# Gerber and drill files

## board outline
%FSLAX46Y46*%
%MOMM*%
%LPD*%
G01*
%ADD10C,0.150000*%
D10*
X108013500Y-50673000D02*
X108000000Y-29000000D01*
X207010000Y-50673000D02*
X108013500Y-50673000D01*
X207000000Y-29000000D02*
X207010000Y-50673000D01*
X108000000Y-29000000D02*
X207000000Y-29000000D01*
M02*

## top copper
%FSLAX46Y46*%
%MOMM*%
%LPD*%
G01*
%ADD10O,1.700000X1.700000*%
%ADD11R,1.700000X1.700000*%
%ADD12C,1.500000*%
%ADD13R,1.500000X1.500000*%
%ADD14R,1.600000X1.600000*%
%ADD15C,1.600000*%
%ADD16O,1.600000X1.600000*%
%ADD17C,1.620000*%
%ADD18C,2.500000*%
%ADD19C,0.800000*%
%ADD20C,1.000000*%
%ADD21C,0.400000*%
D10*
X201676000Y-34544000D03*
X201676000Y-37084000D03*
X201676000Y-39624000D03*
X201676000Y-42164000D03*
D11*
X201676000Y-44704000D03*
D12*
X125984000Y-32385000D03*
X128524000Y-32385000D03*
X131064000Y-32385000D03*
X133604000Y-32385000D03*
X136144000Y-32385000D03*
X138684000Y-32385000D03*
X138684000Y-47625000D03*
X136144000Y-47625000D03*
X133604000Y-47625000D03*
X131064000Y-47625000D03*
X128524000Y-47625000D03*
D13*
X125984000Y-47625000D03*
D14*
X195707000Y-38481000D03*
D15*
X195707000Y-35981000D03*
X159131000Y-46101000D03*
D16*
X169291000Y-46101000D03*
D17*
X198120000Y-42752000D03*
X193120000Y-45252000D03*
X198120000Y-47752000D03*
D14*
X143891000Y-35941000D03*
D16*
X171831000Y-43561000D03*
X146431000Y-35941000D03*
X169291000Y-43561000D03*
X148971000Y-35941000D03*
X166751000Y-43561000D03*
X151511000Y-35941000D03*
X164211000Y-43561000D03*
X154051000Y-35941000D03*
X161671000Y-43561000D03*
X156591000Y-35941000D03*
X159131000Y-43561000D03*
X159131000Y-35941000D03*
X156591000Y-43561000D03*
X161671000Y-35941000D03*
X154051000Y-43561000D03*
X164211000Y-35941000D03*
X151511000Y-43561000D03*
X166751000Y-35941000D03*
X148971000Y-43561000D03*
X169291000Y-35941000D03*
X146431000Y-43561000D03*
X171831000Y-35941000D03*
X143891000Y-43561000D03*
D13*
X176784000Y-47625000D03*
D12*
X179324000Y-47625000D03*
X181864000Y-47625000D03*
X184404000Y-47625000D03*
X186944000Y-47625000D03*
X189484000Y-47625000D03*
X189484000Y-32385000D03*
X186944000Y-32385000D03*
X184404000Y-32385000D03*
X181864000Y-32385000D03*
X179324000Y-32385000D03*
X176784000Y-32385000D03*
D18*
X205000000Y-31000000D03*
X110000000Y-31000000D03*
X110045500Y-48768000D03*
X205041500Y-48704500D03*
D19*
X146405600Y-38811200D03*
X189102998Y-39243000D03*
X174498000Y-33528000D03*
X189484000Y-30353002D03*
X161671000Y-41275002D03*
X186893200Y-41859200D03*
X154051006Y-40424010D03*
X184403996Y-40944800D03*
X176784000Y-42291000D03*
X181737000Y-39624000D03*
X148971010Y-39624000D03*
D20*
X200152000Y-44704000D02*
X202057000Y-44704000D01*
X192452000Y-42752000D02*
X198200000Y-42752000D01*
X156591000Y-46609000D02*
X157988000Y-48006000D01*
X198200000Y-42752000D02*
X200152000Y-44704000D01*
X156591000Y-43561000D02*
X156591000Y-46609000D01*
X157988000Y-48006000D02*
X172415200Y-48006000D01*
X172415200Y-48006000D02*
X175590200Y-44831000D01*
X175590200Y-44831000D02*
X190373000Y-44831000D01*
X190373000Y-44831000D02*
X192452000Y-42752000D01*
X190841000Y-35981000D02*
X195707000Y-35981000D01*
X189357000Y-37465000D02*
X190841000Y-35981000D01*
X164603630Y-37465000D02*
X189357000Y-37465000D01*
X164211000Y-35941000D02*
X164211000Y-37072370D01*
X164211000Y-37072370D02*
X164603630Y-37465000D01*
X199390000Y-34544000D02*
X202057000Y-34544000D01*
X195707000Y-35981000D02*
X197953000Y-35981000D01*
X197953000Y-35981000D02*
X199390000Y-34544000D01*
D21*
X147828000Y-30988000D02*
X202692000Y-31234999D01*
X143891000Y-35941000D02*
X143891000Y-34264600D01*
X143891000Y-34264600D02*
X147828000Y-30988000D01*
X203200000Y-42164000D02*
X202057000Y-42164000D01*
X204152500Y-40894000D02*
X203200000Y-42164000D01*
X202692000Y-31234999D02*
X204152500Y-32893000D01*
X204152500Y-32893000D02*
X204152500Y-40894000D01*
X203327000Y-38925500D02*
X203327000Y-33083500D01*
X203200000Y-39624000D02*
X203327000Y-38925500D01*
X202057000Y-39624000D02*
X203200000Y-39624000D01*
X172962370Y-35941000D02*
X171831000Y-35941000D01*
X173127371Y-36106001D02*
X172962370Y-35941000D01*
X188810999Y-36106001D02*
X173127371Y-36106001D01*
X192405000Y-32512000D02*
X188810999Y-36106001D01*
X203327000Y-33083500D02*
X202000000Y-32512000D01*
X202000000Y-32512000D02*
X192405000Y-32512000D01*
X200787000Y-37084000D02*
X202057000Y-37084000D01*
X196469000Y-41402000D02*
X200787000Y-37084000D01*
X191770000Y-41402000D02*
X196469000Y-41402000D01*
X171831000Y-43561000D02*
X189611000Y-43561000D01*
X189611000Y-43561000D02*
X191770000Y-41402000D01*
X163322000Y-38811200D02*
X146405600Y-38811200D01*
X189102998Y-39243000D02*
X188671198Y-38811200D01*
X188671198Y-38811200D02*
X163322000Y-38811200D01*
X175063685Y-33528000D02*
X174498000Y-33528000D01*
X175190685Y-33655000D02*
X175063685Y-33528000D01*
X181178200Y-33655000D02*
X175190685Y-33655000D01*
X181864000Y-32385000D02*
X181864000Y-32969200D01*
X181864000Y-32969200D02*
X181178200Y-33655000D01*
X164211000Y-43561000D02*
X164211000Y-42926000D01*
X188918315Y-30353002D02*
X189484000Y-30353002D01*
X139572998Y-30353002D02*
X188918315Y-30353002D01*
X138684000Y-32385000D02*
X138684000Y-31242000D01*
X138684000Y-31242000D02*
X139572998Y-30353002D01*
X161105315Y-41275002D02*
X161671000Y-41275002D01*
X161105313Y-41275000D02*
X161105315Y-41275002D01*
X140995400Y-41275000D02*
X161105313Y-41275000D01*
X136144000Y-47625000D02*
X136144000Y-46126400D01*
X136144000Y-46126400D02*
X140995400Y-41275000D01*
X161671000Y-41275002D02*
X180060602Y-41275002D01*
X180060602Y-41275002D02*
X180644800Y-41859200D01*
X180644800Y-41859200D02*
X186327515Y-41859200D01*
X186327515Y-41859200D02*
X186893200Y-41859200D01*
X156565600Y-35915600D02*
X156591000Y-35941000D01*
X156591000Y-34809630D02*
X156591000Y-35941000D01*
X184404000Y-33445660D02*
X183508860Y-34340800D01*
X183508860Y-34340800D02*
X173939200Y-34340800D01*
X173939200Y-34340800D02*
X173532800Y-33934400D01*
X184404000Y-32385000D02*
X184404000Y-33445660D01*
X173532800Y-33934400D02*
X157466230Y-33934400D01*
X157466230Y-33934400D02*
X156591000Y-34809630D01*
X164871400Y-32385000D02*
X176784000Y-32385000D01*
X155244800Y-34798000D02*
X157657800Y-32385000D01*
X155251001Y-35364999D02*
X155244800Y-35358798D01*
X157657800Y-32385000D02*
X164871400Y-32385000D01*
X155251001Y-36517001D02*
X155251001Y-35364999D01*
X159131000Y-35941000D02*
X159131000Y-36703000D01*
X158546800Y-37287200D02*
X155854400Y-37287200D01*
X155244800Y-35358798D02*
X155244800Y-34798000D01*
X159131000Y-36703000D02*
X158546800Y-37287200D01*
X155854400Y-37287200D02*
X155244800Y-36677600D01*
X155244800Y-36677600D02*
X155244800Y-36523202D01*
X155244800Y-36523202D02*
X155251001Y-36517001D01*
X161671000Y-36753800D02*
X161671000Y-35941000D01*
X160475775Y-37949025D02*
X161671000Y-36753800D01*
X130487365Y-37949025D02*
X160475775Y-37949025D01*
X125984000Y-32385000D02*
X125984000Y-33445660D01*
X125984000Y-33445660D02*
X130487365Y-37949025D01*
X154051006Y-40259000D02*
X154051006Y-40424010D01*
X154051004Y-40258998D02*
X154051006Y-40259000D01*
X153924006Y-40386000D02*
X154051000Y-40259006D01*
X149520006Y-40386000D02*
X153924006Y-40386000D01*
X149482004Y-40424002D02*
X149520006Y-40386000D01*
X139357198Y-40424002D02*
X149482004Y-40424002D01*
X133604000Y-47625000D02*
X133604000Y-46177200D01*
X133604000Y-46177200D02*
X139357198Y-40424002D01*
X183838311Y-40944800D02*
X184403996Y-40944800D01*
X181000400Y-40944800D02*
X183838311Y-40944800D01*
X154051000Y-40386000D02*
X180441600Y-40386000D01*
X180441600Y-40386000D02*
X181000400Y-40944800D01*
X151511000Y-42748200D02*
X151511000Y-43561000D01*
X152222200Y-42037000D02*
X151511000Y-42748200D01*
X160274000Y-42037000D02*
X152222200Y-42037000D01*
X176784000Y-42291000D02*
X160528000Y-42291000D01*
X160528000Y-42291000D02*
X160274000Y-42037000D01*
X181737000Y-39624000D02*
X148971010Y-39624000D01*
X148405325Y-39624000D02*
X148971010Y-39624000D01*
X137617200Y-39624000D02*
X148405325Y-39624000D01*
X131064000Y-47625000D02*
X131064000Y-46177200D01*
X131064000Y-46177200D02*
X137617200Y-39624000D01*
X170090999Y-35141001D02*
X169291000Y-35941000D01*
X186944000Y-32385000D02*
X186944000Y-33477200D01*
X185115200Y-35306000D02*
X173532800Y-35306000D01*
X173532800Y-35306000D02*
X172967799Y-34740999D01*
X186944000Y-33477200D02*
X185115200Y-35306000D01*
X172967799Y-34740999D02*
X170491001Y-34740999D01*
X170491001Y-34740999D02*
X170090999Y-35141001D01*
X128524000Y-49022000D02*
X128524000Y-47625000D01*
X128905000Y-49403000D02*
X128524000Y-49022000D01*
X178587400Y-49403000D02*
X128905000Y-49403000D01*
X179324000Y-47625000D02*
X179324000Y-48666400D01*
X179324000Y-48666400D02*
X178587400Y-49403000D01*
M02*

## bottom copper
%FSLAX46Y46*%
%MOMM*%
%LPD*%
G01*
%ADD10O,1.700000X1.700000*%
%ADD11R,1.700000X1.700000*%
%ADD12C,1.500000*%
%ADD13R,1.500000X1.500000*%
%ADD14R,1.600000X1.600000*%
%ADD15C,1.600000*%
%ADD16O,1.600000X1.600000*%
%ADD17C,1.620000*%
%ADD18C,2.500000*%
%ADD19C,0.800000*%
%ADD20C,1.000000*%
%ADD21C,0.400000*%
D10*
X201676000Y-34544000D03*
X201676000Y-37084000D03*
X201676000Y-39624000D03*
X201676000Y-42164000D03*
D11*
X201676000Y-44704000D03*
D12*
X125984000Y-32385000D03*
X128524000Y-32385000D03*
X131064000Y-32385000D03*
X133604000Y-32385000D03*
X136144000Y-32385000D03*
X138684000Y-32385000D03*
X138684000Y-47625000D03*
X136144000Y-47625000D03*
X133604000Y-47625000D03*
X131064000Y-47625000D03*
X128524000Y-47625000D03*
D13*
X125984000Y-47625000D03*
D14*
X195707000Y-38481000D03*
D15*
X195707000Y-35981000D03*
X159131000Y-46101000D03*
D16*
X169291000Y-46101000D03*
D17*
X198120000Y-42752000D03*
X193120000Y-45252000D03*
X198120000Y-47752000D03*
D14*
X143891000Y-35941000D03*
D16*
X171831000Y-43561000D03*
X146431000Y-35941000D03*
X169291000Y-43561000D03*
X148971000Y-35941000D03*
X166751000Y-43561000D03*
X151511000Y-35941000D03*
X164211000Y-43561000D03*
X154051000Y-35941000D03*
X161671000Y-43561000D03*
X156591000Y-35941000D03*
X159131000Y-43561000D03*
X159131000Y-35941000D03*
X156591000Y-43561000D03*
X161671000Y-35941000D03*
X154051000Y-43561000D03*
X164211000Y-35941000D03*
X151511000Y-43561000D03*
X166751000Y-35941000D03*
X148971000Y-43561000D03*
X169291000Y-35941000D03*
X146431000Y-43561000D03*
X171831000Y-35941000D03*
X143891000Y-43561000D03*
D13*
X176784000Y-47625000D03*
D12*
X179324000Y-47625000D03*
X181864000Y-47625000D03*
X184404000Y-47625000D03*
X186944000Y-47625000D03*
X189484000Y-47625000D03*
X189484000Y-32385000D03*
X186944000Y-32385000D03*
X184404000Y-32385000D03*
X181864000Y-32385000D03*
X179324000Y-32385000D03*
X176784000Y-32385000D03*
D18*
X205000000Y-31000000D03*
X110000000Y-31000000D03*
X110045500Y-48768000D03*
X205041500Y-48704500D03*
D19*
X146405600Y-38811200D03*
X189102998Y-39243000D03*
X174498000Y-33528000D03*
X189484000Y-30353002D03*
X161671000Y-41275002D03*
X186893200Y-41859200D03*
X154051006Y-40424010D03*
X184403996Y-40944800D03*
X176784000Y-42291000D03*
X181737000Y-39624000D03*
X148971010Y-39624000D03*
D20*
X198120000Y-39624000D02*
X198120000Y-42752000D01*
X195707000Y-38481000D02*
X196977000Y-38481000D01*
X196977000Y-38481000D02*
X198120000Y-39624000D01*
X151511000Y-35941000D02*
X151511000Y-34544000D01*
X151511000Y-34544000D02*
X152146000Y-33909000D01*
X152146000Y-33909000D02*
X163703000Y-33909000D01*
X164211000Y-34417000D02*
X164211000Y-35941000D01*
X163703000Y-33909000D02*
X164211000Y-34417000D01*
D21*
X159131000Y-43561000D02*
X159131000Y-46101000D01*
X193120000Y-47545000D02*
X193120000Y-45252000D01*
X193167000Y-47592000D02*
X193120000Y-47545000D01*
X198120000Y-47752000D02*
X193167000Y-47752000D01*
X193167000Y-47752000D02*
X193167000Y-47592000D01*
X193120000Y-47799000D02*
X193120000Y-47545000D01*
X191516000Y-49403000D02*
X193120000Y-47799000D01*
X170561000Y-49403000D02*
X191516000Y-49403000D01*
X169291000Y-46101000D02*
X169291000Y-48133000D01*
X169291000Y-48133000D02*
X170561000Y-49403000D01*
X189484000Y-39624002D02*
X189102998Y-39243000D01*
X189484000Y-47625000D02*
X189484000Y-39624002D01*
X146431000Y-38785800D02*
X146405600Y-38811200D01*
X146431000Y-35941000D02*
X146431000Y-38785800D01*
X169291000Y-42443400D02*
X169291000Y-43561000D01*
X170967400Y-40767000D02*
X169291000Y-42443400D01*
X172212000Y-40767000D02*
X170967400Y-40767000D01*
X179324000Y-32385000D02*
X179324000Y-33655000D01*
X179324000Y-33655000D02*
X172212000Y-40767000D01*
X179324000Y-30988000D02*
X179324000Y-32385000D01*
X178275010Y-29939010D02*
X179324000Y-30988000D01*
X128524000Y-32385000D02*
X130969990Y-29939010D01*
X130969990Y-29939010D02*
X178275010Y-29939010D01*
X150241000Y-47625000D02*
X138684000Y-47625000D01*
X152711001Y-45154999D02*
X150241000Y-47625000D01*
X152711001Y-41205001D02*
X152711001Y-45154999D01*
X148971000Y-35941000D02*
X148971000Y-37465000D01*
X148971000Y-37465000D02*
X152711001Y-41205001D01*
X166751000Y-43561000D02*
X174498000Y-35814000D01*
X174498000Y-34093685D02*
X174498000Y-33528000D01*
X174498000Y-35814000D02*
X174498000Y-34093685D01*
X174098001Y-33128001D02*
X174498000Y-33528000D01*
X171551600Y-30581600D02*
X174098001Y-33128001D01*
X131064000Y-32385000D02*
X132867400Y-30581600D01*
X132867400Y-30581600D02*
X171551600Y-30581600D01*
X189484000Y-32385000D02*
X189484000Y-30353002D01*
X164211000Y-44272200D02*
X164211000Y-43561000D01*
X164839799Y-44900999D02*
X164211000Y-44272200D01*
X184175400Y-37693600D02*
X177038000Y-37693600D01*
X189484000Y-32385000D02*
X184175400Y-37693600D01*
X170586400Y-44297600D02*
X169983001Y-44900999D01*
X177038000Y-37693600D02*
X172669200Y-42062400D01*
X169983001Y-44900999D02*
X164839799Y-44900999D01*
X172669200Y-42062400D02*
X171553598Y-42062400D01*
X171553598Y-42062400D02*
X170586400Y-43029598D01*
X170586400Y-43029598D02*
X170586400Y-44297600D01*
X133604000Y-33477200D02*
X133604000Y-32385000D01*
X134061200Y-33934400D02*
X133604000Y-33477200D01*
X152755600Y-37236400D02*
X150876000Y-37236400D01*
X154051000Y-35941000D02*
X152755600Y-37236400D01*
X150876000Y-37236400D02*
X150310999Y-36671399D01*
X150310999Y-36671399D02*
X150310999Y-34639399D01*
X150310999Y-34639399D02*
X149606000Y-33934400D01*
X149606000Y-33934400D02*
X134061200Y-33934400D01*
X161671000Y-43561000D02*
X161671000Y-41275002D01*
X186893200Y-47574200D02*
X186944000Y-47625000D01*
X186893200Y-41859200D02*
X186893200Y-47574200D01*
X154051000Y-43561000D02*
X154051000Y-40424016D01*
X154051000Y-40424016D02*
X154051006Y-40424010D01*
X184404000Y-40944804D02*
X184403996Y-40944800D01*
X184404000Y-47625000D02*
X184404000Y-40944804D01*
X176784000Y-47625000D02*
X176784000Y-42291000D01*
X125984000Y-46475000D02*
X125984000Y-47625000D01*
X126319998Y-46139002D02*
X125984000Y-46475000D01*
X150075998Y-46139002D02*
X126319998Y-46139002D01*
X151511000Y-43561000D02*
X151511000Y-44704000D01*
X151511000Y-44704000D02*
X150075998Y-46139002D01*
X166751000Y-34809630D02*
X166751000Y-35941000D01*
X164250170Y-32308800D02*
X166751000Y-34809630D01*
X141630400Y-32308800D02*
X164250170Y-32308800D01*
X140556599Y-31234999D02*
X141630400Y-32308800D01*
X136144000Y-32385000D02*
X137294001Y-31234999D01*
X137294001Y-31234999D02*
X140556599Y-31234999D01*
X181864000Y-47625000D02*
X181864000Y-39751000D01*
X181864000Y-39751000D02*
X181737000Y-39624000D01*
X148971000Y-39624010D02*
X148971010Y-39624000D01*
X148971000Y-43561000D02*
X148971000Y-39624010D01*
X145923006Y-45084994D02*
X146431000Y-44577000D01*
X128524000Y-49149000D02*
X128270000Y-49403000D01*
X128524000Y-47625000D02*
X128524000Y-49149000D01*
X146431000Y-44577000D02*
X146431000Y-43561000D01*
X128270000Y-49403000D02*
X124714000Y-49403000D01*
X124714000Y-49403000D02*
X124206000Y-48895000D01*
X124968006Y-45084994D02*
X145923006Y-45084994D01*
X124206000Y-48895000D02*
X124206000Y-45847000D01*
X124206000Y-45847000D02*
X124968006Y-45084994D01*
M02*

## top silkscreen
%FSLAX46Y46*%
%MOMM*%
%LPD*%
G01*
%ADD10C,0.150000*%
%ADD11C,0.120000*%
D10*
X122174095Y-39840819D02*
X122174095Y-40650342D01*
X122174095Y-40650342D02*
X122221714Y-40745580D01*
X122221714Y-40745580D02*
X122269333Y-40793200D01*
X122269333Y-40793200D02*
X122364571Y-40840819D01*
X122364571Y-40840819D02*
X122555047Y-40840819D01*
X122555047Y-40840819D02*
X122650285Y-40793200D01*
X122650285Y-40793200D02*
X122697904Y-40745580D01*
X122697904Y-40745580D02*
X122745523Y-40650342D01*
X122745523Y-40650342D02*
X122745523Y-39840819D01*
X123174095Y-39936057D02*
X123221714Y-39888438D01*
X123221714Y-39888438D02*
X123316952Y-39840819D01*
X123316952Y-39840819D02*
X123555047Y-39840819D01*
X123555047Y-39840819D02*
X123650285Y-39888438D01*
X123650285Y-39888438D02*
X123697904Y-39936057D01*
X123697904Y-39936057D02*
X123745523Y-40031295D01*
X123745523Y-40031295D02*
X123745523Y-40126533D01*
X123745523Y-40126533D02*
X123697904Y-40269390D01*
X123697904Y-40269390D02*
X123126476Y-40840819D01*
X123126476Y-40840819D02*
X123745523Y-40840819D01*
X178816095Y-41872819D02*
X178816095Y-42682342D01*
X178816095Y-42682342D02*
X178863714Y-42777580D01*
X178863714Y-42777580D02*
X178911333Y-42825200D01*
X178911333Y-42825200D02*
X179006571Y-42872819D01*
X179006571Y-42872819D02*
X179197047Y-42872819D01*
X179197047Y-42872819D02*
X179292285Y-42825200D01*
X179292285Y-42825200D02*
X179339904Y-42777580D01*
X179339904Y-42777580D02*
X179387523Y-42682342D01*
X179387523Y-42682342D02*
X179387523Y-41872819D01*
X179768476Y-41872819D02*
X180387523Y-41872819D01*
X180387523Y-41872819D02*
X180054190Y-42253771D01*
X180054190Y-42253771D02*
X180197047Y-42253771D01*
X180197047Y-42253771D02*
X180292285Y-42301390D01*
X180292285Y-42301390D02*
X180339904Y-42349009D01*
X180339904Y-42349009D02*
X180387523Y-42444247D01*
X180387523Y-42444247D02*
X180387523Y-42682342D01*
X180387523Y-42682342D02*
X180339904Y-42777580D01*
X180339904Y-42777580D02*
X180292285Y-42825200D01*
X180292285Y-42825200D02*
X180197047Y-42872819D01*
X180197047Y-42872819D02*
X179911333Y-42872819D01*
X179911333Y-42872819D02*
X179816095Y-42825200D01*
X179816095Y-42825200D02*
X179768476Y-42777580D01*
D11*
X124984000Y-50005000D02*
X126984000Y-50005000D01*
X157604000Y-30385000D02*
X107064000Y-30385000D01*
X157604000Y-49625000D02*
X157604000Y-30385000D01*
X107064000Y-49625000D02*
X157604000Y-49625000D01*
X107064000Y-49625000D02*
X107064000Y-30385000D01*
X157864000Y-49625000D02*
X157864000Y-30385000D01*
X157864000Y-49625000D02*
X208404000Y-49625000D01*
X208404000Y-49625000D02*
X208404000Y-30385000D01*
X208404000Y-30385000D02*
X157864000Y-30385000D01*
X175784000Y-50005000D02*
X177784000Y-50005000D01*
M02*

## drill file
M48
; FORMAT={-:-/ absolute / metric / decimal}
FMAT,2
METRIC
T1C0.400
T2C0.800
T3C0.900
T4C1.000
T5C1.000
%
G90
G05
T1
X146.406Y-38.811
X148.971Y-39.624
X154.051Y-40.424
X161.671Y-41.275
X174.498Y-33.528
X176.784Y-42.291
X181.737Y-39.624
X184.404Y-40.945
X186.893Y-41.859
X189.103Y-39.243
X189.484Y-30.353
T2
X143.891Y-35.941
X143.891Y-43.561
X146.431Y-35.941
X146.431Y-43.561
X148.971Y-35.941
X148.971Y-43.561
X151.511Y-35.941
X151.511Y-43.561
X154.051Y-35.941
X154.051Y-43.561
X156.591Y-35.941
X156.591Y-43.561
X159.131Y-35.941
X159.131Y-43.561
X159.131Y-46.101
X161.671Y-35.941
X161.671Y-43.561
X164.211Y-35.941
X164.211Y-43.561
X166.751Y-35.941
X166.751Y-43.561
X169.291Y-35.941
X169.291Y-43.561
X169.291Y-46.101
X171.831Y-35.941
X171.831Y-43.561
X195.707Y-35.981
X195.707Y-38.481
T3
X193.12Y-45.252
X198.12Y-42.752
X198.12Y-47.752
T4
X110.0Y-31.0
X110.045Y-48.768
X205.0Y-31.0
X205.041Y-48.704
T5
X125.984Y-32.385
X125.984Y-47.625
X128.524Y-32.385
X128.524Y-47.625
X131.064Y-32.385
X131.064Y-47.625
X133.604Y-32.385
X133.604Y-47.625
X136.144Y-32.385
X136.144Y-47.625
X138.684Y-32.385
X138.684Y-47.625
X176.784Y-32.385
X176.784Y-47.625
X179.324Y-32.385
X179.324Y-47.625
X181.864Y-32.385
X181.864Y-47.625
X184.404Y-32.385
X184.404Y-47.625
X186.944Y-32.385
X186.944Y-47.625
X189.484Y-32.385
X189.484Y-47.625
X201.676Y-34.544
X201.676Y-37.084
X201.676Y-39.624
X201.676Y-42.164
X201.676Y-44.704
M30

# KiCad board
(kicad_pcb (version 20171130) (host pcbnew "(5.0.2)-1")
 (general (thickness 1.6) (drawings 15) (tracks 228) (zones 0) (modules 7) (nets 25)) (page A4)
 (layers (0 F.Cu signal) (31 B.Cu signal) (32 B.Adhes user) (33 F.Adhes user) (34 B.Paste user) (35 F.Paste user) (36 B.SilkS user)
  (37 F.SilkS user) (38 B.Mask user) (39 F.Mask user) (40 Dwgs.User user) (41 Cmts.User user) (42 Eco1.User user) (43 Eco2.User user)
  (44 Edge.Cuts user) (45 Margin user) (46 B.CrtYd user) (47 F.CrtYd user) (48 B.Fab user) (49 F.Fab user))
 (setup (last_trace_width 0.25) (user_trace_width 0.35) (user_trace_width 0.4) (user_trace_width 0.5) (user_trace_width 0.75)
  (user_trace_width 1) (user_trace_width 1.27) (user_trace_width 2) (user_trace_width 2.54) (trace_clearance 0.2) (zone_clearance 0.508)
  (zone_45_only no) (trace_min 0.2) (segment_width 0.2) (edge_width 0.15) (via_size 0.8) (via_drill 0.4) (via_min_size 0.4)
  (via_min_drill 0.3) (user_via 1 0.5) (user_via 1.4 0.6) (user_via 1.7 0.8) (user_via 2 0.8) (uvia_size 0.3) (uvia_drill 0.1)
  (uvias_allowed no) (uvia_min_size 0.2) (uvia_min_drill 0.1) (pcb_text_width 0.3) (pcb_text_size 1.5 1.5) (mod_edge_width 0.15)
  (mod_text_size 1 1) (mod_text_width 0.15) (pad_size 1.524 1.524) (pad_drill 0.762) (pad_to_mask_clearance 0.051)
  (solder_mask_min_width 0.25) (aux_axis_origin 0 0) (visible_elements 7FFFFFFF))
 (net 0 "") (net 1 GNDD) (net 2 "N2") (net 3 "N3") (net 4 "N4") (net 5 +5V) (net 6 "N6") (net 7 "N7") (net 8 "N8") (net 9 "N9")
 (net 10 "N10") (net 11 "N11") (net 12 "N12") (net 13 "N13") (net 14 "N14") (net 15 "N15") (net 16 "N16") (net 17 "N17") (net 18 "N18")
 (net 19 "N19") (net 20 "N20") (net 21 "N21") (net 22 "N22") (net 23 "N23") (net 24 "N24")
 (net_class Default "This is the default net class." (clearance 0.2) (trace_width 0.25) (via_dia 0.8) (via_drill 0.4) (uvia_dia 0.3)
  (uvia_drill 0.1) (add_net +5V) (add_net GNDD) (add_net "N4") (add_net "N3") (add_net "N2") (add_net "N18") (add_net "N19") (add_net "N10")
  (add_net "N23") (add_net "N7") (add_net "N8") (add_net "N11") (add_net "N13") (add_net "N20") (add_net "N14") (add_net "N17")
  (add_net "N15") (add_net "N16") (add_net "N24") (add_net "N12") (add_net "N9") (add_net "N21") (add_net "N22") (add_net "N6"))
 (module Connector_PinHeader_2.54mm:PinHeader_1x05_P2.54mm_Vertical (layer B.Cu) (at 201.676 44.704)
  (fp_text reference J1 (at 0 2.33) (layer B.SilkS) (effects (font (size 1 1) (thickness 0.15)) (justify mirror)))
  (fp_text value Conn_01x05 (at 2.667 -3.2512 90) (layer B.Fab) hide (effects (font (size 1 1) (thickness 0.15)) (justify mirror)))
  (pad 5 thru_hole oval (at 0 -10.16) (size 1.7 1.7) (drill 1) (layers *.Cu *.Mask) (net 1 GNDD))
  (pad 4 thru_hole oval (at 0 -7.62) (size 1.7 1.7) (drill 1) (layers *.Cu *.Mask) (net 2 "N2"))
  (pad 3 thru_hole oval (at 0 -5.08) (size 1.7 1.7) (drill 1) (layers *.Cu *.Mask) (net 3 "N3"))
  (pad 2 thru_hole oval (at 0 -2.54) (size 1.7 1.7) (drill 1) (layers *.Cu *.Mask) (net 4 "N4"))
  (pad 1 thru_hole rect (at 0 0) (size 1.7 1.7) (drill 1) (layers *.Cu *.Mask) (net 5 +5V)))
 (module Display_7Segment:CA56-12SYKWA (layer F.Cu) (at 125.984 47.625 90)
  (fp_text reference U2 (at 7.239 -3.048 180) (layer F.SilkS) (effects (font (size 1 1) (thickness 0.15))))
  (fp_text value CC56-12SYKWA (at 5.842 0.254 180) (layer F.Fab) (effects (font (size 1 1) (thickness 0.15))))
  (fp_line (start -2.38 -1) (end -2.38 1) (layer F.SilkS) (width 0.12))
  (fp_line (start 17.24 31.62) (end 17.24 -18.92) (layer F.SilkS) (width 0.12))
  (fp_line (start -2 31.62) (end 17.24 31.62) (layer F.SilkS) (width 0.12))
  (fp_line (start -2 -18.92) (end -2 31.62) (layer F.SilkS) (width 0.12))
  (fp_line (start -2 -18.92) (end 17.24 -18.92) (layer F.SilkS) (width 0.12))
  (pad 12 thru_hole circle (at 15.24 0 90) (size 1.5 1.5) (drill 1) (layers *.Cu *.Mask) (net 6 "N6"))
  (pad 11 thru_hole circle (at 15.24 2.54 90) (size 1.5 1.5) (drill 1) (layers *.Cu *.Mask) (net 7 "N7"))
  (pad 10 thru_hole circle (at 15.24 5.08 90) (size 1.5 1.5) (drill 1) (layers *.Cu *.Mask) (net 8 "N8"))
  (pad 9 thru_hole circle (at 15.24 7.62 90) (size 1.5 1.5) (drill 1) (layers *.Cu *.Mask) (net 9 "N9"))
  (pad 8 thru_hole circle (at 15.24 10.16 90) (size 1.5 1.5) (drill 1) (layers *.Cu *.Mask) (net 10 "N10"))
  (pad 7 thru_hole circle (at 15.24 12.7 90) (size 1.5 1.5) (drill 1) (layers *.Cu *.Mask) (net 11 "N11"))
  (pad 6 thru_hole circle (at 0 12.7 90) (size 1.5 1.5) (drill 1) (layers *.Cu *.Mask) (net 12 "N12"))
  (pad 5 thru_hole circle (at 0 10.16 90) (size 1.5 1.5) (drill 1) (layers *.Cu *.Mask) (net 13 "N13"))
  (pad 4 thru_hole circle (at 0 7.62 90) (size 1.5 1.5) (drill 1) (layers *.Cu *.Mask) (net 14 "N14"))
  (pad 3 thru_hole circle (at 0 5.08 90) (size 1.5 1.5) (drill 1) (layers *.Cu *.Mask) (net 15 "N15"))
  (pad 2 thru_hole circle (at 0 2.54 90) (size 1.5 1.5) (drill 1) (layers *.Cu *.Mask) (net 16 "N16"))
  (pad 1 thru_hole rect (at 0 0 90) (size 1.5 1.5) (drill 1) (layers *.Cu *.Mask) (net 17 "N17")))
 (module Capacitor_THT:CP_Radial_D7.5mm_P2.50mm (layer B.Cu) (at 195.707 38.481 90)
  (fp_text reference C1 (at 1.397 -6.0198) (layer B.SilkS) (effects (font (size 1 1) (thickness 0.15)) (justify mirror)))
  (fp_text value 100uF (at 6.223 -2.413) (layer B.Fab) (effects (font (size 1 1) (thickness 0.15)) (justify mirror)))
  (pad 1 thru_hole rect (at 0 0 90) (size 1.6 1.6) (drill 0.8) (layers *.Cu *.Mask) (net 5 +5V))
  (pad 2 thru_hole circle (at 2.5 0 90) (size 1.6 1.6) (drill 0.8) (layers *.Cu *.Mask) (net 1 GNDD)))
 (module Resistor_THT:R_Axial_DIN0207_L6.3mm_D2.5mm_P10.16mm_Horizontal (layer B.Cu) (at 159.131 46.101)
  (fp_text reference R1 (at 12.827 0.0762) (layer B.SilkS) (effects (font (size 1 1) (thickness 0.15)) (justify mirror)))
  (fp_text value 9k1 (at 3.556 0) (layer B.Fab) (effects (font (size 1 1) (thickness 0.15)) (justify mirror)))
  (pad 1 thru_hole circle (at 0 0) (size 1.6 1.6) (drill 0.8) (layers *.Cu *.Mask) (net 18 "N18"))
  (pad 2 thru_hole oval (at 10.16 0) (size 1.6 1.6) (drill 0.8) (layers *.Cu *.Mask) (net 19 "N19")))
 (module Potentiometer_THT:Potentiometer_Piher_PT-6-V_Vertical (layer B.Cu) (at 198.12 47.752 180)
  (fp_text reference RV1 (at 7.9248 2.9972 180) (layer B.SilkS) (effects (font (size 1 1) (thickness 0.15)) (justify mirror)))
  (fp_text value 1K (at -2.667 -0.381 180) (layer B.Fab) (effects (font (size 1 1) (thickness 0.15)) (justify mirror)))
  (pad 3 thru_hole circle (at 0 5 180) (size 1.62 1.62) (drill 0.9) (layers *.Cu *.Mask) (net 5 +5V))
  (pad 2 thru_hole circle (at 5 2.5 180) (size 1.62 1.62) (drill 0.9) (layers *.Cu *.Mask) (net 19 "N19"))
  (pad 1 thru_hole circle (at 0 0 180) (size 1.62 1.62) (drill 0.9) (layers *.Cu *.Mask) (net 19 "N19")))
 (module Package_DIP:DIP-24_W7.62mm (layer B.Cu) (at 143.891 35.941 270)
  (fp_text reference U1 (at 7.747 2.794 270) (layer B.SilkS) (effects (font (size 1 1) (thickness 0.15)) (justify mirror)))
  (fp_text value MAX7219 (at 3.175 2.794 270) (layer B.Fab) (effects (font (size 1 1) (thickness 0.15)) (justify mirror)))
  (pad 1 thru_hole rect (at 0 0 270) (size 1.6 1.6) (drill 0.8) (layers *.Cu *.Mask) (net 4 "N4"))
  (pad 13 thru_hole oval (at 7.62 -27.94 270) (size 1.6 1.6) (drill 0.8) (layers *.Cu *.Mask) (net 2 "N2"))
  (pad 2 thru_hole oval (at 0 -2.54 270) (size 1.6 1.6) (drill 0.8) (layers *.Cu *.Mask) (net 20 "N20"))
  (pad 14 thru_hole oval (at 7.62 -25.4 270) (size 1.6 1.6) (drill 0.8) (layers *.Cu *.Mask) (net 7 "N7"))
  (pad 3 thru_hole oval (at 0 -5.08 270) (size 1.6 1.6) (drill 0.8) (layers *.Cu *.Mask) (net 12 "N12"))
  (pad 15 thru_hole oval (at 7.62 -22.86 270) (size 1.6 1.6) (drill 0.8) (layers *.Cu *.Mask) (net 8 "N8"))
  (pad 4 thru_hole oval (at 0 -7.62 270) (size 1.6 1.6) (drill 0.8) (layers *.Cu *.Mask) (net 1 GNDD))
  (pad 16 thru_hole oval (at 7.62 -20.32 270) (size 1.6 1.6) (drill 0.8) (layers *.Cu *.Mask) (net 11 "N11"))
  (pad 5 thru_hole oval (at 0 -10.16 270) (size 1.6 1.6) (drill 0.8) (layers *.Cu *.Mask) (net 9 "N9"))
  (pad 17 thru_hole oval (at 7.62 -17.78 270) (size 1.6 1.6) (drill 0.8) (layers *.Cu *.Mask) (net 13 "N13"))
  (pad 6 thru_hole oval (at 0 -12.7 270) (size 1.6 1.6) (drill 0.8) (layers *.Cu *.Mask) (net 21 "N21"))
  (pad 18 thru_hole oval (at 7.62 -15.24 270) (size 1.6 1.6) (drill 0.8) (layers *.Cu *.Mask) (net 18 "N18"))
  (pad 7 thru_hole oval (at 0 -15.24 270) (size 1.6 1.6) (drill 0.8) (layers *.Cu *.Mask) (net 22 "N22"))
  (pad 19 thru_hole oval (at 7.62 -12.7 270) (size 1.6 1.6) (drill 0.8) (layers *.Cu *.Mask) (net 5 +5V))
  (pad 8 thru_hole oval (at 0 -17.78 270) (size 1.6 1.6) (drill 0.8) (layers *.Cu *.Mask) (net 6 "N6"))
  (pad 20 thru_hole oval (at 7.62 -10.16 270) (size 1.6 1.6) (drill 0.8) (layers *.Cu *.Mask) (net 14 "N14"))
  (pad 9 thru_hole oval (at 0 -20.32 270) (size 1.6 1.6) (drill 0.8) (layers *.Cu *.Mask) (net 1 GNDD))
  (pad 21 thru_hole oval (at 7.62 -7.62 270) (size 1.6 1.6) (drill 0.8) (layers *.Cu *.Mask) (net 17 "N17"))
  (pad 10 thru_hole oval (at 0 -22.86 270) (size 1.6 1.6) (drill 0.8) (layers *.Cu *.Mask) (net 10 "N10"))
  (pad 22 thru_hole oval (at 7.62 -5.08 270) (size 1.6 1.6) (drill 0.8) (layers *.Cu *.Mask) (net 15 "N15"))
  (pad 11 thru_hole oval (at 0 -25.4 270) (size 1.6 1.6) (drill 0.8) (layers *.Cu *.Mask) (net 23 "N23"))
  (pad 23 thru_hole oval (at 7.62 -2.54 270) (size 1.6 1.6) (drill 0.8) (layers *.Cu *.Mask) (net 16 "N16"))
  (pad 12 thru_hole oval (at 0 -27.94 270) (size 1.6 1.6) (drill 0.8) (layers *.Cu *.Mask) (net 3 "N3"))
  (pad 24 thru_hole oval (at 7.62 0 270) (size 1.6 1.6) (drill 0.8) (layers *.Cu *.Mask) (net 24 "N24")))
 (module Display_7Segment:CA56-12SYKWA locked (layer F.Cu) (at 176.784 47.625 90)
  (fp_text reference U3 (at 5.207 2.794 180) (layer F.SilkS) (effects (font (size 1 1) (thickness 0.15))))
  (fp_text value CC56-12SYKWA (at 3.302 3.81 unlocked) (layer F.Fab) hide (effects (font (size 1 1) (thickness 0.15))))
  (fp_line (start -2 -18.92) (end 17.24 -18.92) (layer F.SilkS) (width 0.12))
  (fp_line (start -2 -18.92) (end -2 31.62) (layer F.SilkS) (width 0.12))
  (fp_line (start -2 31.62) (end 17.24 31.62) (layer F.SilkS) (width 0.12))
  (fp_line (start 17.24 31.62) (end 17.24 -18.92) (layer F.SilkS) (width 0.12))
  (fp_line (start -2.38 -1) (end -2.38 1) (layer F.SilkS) (width 0.12))
  (pad 1 thru_hole rect (at 0 0 90) (size 1.5 1.5) (drill 1) (layers *.Cu *.Mask) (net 17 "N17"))
  (pad 2 thru_hole circle (at 0 2.54 90) (size 1.5 1.5) (drill 1) (layers *.Cu *.Mask) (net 16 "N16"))
  (pad 3 thru_hole circle (at 0 5.08 90) (size 1.5 1.5) (drill 1) (layers *.Cu *.Mask) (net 15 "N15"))
  (pad 4 thru_hole circle (at 0 7.62 90) (size 1.5 1.5) (drill 1) (layers *.Cu *.Mask) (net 14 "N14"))
  (pad 5 thru_hole circle (at 0 10.16 90) (size 1.5 1.5) (drill 1) (layers *.Cu *.Mask) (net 13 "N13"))
  (pad 6 thru_hole circle (at 0 12.7 90) (size 1.5 1.5) (drill 1) (layers *.Cu *.Mask) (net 20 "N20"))
  (pad 7 thru_hole circle (at 15.24 12.7 90) (size 1.5 1.5) (drill 1) (layers *.Cu *.Mask) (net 11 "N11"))
  (pad 8 thru_hole circle (at 15.24 10.16 90) (size 1.5 1.5) (drill 1) (layers *.Cu *.Mask) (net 23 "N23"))
  (pad 9 thru_hole circle (at 15.24 7.62 90) (size 1.5 1.5) (drill 1) (layers *.Cu *.Mask) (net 21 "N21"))
  (pad 10 thru_hole circle (at 15.24 5.08 90) (size 1.5 1.5) (drill 1) (layers *.Cu *.Mask) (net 8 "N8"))
  (pad 11 thru_hole circle (at 15.24 2.54 90) (size 1.5 1.5) (drill 1) (layers *.Cu *.Mask) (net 7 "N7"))
  (pad 12 thru_hole circle (at 15.24 0 90) (size 1.5 1.5) (drill 1) (layers *.Cu *.Mask) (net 22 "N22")))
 (gr_line (start 108.0135 50.673) (end 108 29) (layer Edge.Cuts) (width 0.15))
 (gr_line (start 207.01 50.673) (end 108.0135 50.673) (layer Edge.Cuts) (width 0.15))
 (gr_line (start 207 29) (end 207.01 50.673) (layer Edge.Cuts) (width 0.15))
 (gr_line (start 108 29) (end 207 29) (layer Edge.Cuts) (width 0.15))
 (via (at 205 31) (size 2.5) (drill 1) (layers F.Cu B.Cu) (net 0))
 (via (at 110 31) (size 2.5) (drill 1) (layers F.Cu B.Cu) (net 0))
 (via (at 110.0455 48.768) (size 2.5) (drill 1) (layers F.Cu B.Cu) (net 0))
 (via (at 205.0415 48.7045) (size 2.5) (drill 1) (layers F.Cu B.Cu) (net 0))
 (segment (start 198.12 39.624) (end 198.12 42.752) (width 1) (layer B.Cu) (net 5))
 (segment (start 195.707 38.481) (end 196.977 38.481) (width 1) (layer B.Cu) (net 5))
 (segment (start 196.977 38.481) (end 198.12 39.624) (width 1) (layer B.Cu) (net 5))
 (segment (start 200.152 44.704) (end 202.057 44.704) (width 1) (layer F.Cu) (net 5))
 (segment (start 192.452 42.752) (end 198.2 42.752) (width 1) (layer F.Cu) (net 5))
 (segment (start 156.591 46.609) (end 157.988 48.006) (width 1) (layer F.Cu) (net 5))
 (segment (start 198.2 42.752) (end 200.152 44.704) (width 1) (layer F.Cu) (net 5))
 (segment (start 156.591 43.561) (end 156.591 46.609) (width 1) (layer F.Cu) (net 5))
 (segment (start 157.988 48.006) (end 172.4152 48.006) (width 1) (layer F.Cu) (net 5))
 (segment (start 172.4152 48.006) (end 175.5902 44.831) (width 1) (layer F.Cu) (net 5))
 (segment (start 175.5902 44.831) (end 190.373 44.831) (width 1) (layer F.Cu) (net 5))
 (segment (start 190.373 44.831) (end 192.452 42.752) (width 1) (layer F.Cu) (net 5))
 (segment (start 151.511 35.941) (end 151.511 34.544) (width 1) (layer B.Cu) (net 1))
 (segment (start 151.511 34.544) (end 152.146 33.909) (width 1) (layer B.Cu) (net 1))
 (segment (start 152.146 33.909) (end 163.703 33.909) (width 1) (layer B.Cu) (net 1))
 (segment (start 164.211 34.417) (end 164.211 35.941) (width 1) (layer B.Cu) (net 1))
 (segment (start 163.703 33.909) (end 164.211 34.417) (width 1) (layer B.Cu) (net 1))
 (segment (start 190.841 35.981) (end 195.707 35.981) (width 1) (layer F.Cu) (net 1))
 (segment (start 189.357 37.465) (end 190.841 35.981) (width 1) (layer F.Cu) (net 1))
 (segment (start 164.60363 37.465) (end 189.357 37.465) (width 1) (layer F.Cu) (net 1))
 (segment (start 164.211 35.941) (end 164.211 37.07237) (width 1) (layer F.Cu) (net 1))
 (segment (start 164.211 37.07237) (end 164.60363 37.465) (width 1) (layer F.Cu) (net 1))
 (segment (start 199.39 34.544) (end 202.057 34.544) (width 1) (layer F.Cu) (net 1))
 (segment (start 195.707 35.981) (end 197.953 35.981) (width 1) (layer F.Cu) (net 1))
 (segment (start 197.953 35.981) (end 199.39 34.544) (width 1) (layer F.Cu) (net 1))
 (segment (start 147.828 30.988) (end 202.692 31.234999) (width 0.4) (layer F.Cu) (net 4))
 (segment (start 143.891 35.941) (end 143.891 34.2646) (width 0.4) (layer F.Cu) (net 4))
 (segment (start 143.891 34.2646) (end 147.828 30.988) (width 0.4) (layer F.Cu) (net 4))
 (segment (start 203.2 42.164) (end 202.057 42.164) (width 0.4) (layer F.Cu) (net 4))
 (segment (start 204.1525 40.894) (end 203.2 42.164) (width 0.4) (layer F.Cu) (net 4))
 (segment (start 202.692 31.234999) (end 204.1525 32.893) (width 0.4) (layer F.Cu) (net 4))
 (segment (start 204.1525 32.893) (end 204.1525 40.894) (width 0.4) (layer F.Cu) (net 4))
 (segment (start 203.327 38.9255) (end 203.327 33.0835) (width 0.4) (layer F.Cu) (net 3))
 (segment (start 203.2 39.624) (end 203.327 38.9255) (width 0.4) (layer F.Cu) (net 3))
 (segment (start 202.057 39.624) (end 203.2 39.624) (width 0.4) (layer F.Cu) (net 3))
 (segment (start 172.96237 35.941) (end 171.831 35.941) (width 0.4) (layer F.Cu) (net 3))
 (segment (start 173.127371 36.106001) (end 172.96237 35.941) (width 0.4) (layer F.Cu) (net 3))
 (segment (start 188.810999 36.106001) (end 173.127371 36.106001) (width 0.4) (layer F.Cu) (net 3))
 (segment (start 192.405 32.512) (end 188.810999 36.106001) (width 0.4) (layer F.Cu) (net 3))
 (segment (start 203.327 33.0835) (end 202 32.512) (width 0.4) (layer F.Cu) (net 3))
 (segment (start 202 32.512) (end 192.405 32.512) (width 0.4) (layer F.Cu) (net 3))
 (segment (start 200.787 37.084) (end 202.057 37.084) (width 0.4) (layer F.Cu) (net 2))
 (segment (start 196.469 41.402) (end 200.787 37.084) (width 0.4) (layer F.Cu) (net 2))
 (segment (start 191.77 41.402) (end 196.469 41.402) (width 0.4) (layer F.Cu) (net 2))
 (segment (start 171.831 43.561) (end 189.611 43.561) (width 0.4) (layer F.Cu) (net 2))
 (segment (start 189.611 43.561) (end 191.77 41.402) (width 0.4) (layer F.Cu) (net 2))
 (segment (start 159.131 43.561) (end 159.131 46.101) (width 0.4) (layer B.Cu) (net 18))
 (segment (start 193.12 47.545) (end 193.12 45.252) (width 0.4) (layer B.Cu) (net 19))
 (segment (start 193.167 47.592) (end 193.12 47.545) (width 0.4) (layer B.Cu) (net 19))
 (segment (start 198.12 47.752) (end 193.167 47.752) (width 0.4) (layer B.Cu) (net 19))
 (segment (start 193.167 47.752) (end 193.167 47.592) (width 0.4) (layer B.Cu) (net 19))
 (segment (start 193.12 47.799) (end 193.12 47.545) (width 0.4) (layer B.Cu) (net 19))
 (segment (start 191.516 49.403) (end 193.12 47.799) (width 0.4) (layer B.Cu) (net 19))
 (segment (start 170.561 49.403) (end 191.516 49.403) (width 0.4) (layer B.Cu) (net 19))
 (segment (start 169.291 46.101) (end 169.291 48.133) (width 0.4) (layer B.Cu) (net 19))
 (segment (start 169.291 48.133) (end 170.561 49.403) (width 0.4) (layer B.Cu) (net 19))
 (via (at 146.4056 38.8112) (size 0.8) (drill 0.4) (layers F.Cu B.Cu) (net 20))
 (segment (start 189.484 39.624002) (end 189.102998 39.243) (width 0.4) (layer B.Cu) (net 20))
 (segment (start 189.484 47.625) (end 189.484 39.624002) (width 0.4) (layer B.Cu) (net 20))
 (via (at 189.102998 39.243) (size 0.8) (drill 0.4) (layers F.Cu B.Cu) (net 20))
 (segment (start 146.431 38.7858) (end 146.4056 38.8112) (width 0.4) (layer B.Cu) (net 20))
 (segment (start 146.431 35.941) (end 146.431 38.7858) (width 0.4) (layer B.Cu) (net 20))
 (segment (start 163.322 38.8112) (end 146.4056 38.8112) (width 0.4) (layer F.Cu) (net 20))
 (segment (start 189.102998 39.243) (end 188.671198 38.8112) (width 0.4) (layer F.Cu) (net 20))
 (segment (start 188.671198 38.8112) (end 163.322 38.8112) (width 0.4) (layer F.Cu) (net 20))
 (segment (start 169.291 42.4434) (end 169.291 43.561) (width 0.4) (layer B.Cu) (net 7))
 (segment (start 170.9674 40.767) (end 169.291 42.4434) (width 0.4) (layer B.Cu) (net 7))
 (segment (start 172.212 40.767) (end 170.9674 40.767) (width 0.4) (layer B.Cu) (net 7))
 (segment (start 179.324 32.385) (end 179.324 33.655) (width 0.4) (layer B.Cu) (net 7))
 (segment (start 179.324 33.655) (end 172.212 40.767) (width 0.4) (layer B.Cu) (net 7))
 (segment (start 179.324 30.988) (end 179.324 32.385) (width 0.4) (layer B.Cu) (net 7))
 (segment (start 178.27501 29.93901) (end 179.324 30.988) (width 0.4) (layer B.Cu) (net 7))
 (segment (start 128.524 32.385) (end 130.96999 29.93901) (width 0.4) (layer B.Cu) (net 7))
 (segment (start 130.96999 29.93901) (end 178.27501 29.93901) (width 0.4) (layer B.Cu) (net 7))
 (segment (start 150.241 47.625) (end 138.684 47.625) (width 0.4) (layer B.Cu) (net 12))
 (segment (start 152.711001 45.154999) (end 150.241 47.625) (width 0.4) (layer B.Cu) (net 12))
 (segment (start 152.711001 41.205001) (end 152.711001 45.154999) (width 0.4) (layer B.Cu) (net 12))
 (segment (start 148.971 35.941) (end 148.971 37.465) (width 0.4) (layer B.Cu) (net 12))
 (segment (start 148.971 37.465) (end 152.711001 41.205001) (width 0.4) (layer B.Cu) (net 12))
 (segment (start 166.751 43.561) (end 174.498 35.814) (width 0.4) (layer B.Cu) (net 8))
 (segment (start 174.498 34.093685) (end 174.498 33.528) (width 0.4) (layer B.Cu) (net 8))
 (segment (start 174.498 35.814) (end 174.498 34.093685) (width 0.4) (layer B.Cu) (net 8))
 (via (at 174.498 33.528) (size 0.8) (drill 0.4) (layers F.Cu B.Cu) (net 8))
 (segment (start 175.063685 33.528) (end 174.498 33.528) (width 0.4) (layer F.Cu) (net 8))
 (segment (start 175.190685 33.655) (end 175.063685 33.528) (width 0.4) (layer F.Cu) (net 8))
 (segment (start 181.1782 33.655) (end 175.190685 33.655) (width 0.4) (layer F.Cu) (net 8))
 (segment (start 181.864 32.385) (end 181.864 32.9692) (width 0.4) (layer F.Cu) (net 8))
 (segment (start 181.864 32.9692) (end 181.1782 33.655) (width 0.4) (layer F.Cu) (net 8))
 (segment (start 174.098001 33.128001) (end 174.498 33.528) (width 0.4) (layer B.Cu) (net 8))
 (segment (start 171.5516 30.5816) (end 174.098001 33.128001) (width 0.4) (layer B.Cu) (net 8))
 (segment (start 131.064 32.385) (end 132.8674 30.5816) (width 0.4) (layer B.Cu) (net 8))
 (segment (start 132.8674 30.5816) (end 171.5516 30.5816) (width 0.4) (layer B.Cu) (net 8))
 (segment (start 164.211 43.561) (end 164.211 42.926) (width 0.4) (layer F.Cu) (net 11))
 (segment (start 189.484 32.385) (end 189.484 30.353002) (width 0.4) (layer B.Cu) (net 11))
 (via (at 189.484 30.353002) (size 0.8) (drill 0.4) (layers F.Cu B.Cu) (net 11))
 (segment (start 188.918315 30.353002) (end 189.484 30.353002) (width 0.4) (layer F.Cu) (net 11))
 (segment (start 139.572998 30.353002) (end 188.918315 30.353002) (width 0.4) (layer F.Cu) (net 11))
 (segment (start 138.684 32.385) (end 138.684 31.242) (width 0.4) (layer F.Cu) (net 11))
 (segment (start 138.684 31.242) (end 139.572998 30.353002) (width 0.4) (layer F.Cu) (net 11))
 (segment (start 164.211 44.2722) (end 164.211 43.561) (width 0.4) (layer B.Cu) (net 11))
 (segment (start 164.839799 44.900999) (end 164.211 44.2722) (width 0.4) (layer B.Cu) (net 11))
 (segment (start 184.1754 37.6936) (end 177.038 37.6936) (width 0.4) (layer B.Cu) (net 11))
 (segment (start 189.484 32.385) (end 184.1754 37.6936) (width 0.4) (layer B.Cu) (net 11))
 (segment (start 170.5864 44.2976) (end 169.983001 44.900999) (width 0.4) (layer B.Cu) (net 11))
 (segment (start 177.038 37.6936) (end 172.6692 42.0624) (width 0.4) (layer B.Cu) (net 11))
 (segment (start 169.983001 44.900999) (end 164.839799 44.900999) (width 0.4) (layer B.Cu) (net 11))
 (segment (start 172.6692 42.0624) (end 171.553598 42.0624) (width 0.4) (layer B.Cu) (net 11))
 (segment (start 171.553598 42.0624) (end 170.5864 43.029598) (width 0.4) (layer B.Cu) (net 11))
 (segment (start 170.5864 43.029598) (end 170.5864 44.2976) (width 0.4) (layer B.Cu) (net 11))
 (segment (start 133.604 33.4772) (end 133.604 32.385) (width 0.4) (layer B.Cu) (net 9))
 (segment (start 134.0612 33.9344) (end 133.604 33.4772) (width 0.4) (layer B.Cu) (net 9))
 (segment (start 152.7556 37.2364) (end 150.876 37.2364) (width 0.4) (layer B.Cu) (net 9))
 (segment (start 154.051 35.941) (end 152.7556 37.2364) (width 0.4) (layer B.Cu) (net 9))
 (segment (start 150.876 37.2364) (end 150.310999 36.671399) (width 0.4) (layer B.Cu) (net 9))
 (segment (start 150.310999 36.671399) (end 150.310999 34.639399) (width 0.4) (layer B.Cu) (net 9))
 (segment (start 150.310999 34.639399) (end 149.606 33.9344) (width 0.4) (layer B.Cu) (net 9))
 (segment (start 149.606 33.9344) (end 134.0612 33.9344) (width 0.4) (layer B.Cu) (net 9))
 (via (at 161.671 41.275002) (size 0.8) (drill 0.4) (layers F.Cu B.Cu) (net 13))
 (segment (start 161.671 43.561) (end 161.671 41.275002) (width 0.4) (layer B.Cu) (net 13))
 (segment (start 161.105315 41.275002) (end 161.671 41.275002) (width 0.4) (layer F.Cu) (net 13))
 (segment (start 161.105313 41.275) (end 161.105315 41.275002) (width 0.4) (layer F.Cu) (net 13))
 (segment (start 140.9954 41.275) (end 161.105313 41.275) (width 0.4) (layer F.Cu) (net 13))
 (segment (start 136.144 47.625) (end 136.144 46.1264) (width 0.4) (layer F.Cu) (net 13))
 (segment (start 136.144 46.1264) (end 140.9954 41.275) (width 0.4) (layer F.Cu) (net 13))
 (via (at 186.8932 41.8592) (size 0.8) (drill 0.4) (layers F.Cu B.Cu) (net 13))
 (segment (start 186.8932 47.5742) (end 186.944 47.625) (width 0.4) (layer B.Cu) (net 13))
 (segment (start 186.8932 41.8592) (end 186.8932 47.5742) (width 0.4) (layer B.Cu) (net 13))
 (segment (start 161.671 41.275002) (end 180.060602 41.275002) (width 0.4) (layer F.Cu) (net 13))
 (segment (start 180.060602 41.275002) (end 180.6448 41.8592) (width 0.4) (layer F.Cu) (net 13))
 (segment (start 180.6448 41.8592) (end 186.327515 41.8592) (width 0.4) (layer F.Cu) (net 13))
 (segment (start 186.327515 41.8592) (end 186.8932 41.8592) (width 0.4) (layer F.Cu) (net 13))
 (segment (start 156.5656 35.9156) (end 156.591 35.941) (width 0.4) (layer F.Cu) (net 21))
 (segment (start 156.591 34.80963) (end 156.591 35.941) (width 0.4) (layer F.Cu) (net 21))
 (segment (start 184.404 33.44566) (end 183.50886 34.3408) (width 0.4) (layer F.Cu) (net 21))
 (segment (start 183.50886 34.3408) (end 173.9392 34.3408) (width 0.4) (layer F.Cu) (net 21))
 (segment (start 173.9392 34.3408) (end 173.5328 33.9344) (width 0.4) (layer F.Cu) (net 21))
 (segment (start 184.404 32.385) (end 184.404 33.44566) (width 0.4) (layer F.Cu) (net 21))
 (segment (start 173.5328 33.9344) (end 157.46623 33.9344) (width 0.4) (layer F.Cu) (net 21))
 (segment (start 157.46623 33.9344) (end 156.591 34.80963) (width 0.4) (layer F.Cu) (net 21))
 (segment (start 164.8714 32.385) (end 176.784 32.385) (width 0.4) (layer F.Cu) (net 22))
 (segment (start 155.2448 34.798) (end 157.6578 32.385) (width 0.4) (layer F.Cu) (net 22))
 (segment (start 155.251001 35.364999) (end 155.2448 35.358798) (width 0.4) (layer F.Cu) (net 22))
 (segment (start 157.6578 32.385) (end 164.8714 32.385) (width 0.4) (layer F.Cu) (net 22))
 (segment (start 155.251001 36.517001) (end 155.251001 35.364999) (width 0.4) (layer F.Cu) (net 22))
 (segment (start 159.131 35.941) (end 159.131 36.703) (width 0.4) (layer F.Cu) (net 22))
 (segment (start 158.5468 37.2872) (end 155.8544 37.2872) (width 0.4) (layer F.Cu) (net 22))
 (segment (start 155.2448 35.358798) (end 155.2448 34.798) (width 0.4) (layer F.Cu) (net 22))
 (segment (start 159.131 36.703) (end 158.5468 37.2872) (width 0.4) (layer F.Cu) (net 22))
 (segment (start 155.8544 37.2872) (end 155.2448 36.6776) (width 0.4) (layer F.Cu) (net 22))
 (segment (start 155.2448 36.6776) (end 155.2448 36.523202) (width 0.4) (layer F.Cu) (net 22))
 (segment (start 155.2448 36.523202) (end 155.251001 36.517001) (width 0.4) (layer F.Cu) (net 22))
 (segment (start 161.671 36.7538) (end 161.671 35.941) (width 0.4) (layer F.Cu) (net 6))
 (segment (start 160.475775 37.949025) (end 161.671 36.7538) (width 0.4) (layer F.Cu) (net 6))
 (segment (start 130.487365 37.949025) (end 160.475775 37.949025) (width 0.4) (layer F.Cu) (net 6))
 (segment (start 125.984 32.385) (end 125.984 33.44566) (width 0.4) (layer F.Cu) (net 6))
 (segment (start 125.984 33.44566) (end 130.487365 37.949025) (width 0.4) (layer F.Cu) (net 6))
 (segment (start 154.051006 40.259) (end 154.051006 40.42401) (width 0.4) (layer F.Cu) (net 14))
 (segment (start 154.051 43.561) (end 154.051 40.424016) (width 0.4) (layer B.Cu) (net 14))
 (segment (start 154.051 40.424016) (end 154.051006 40.42401) (width 0.4) (layer B.Cu) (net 14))
 (via (at 154.051006 40.42401) (size 0.8) (drill 0.4) (layers F.Cu B.Cu) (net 14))
 (segment (start 154.051004 40.258998) (end 154.051006 40.259) (width 0.4) (layer F.Cu) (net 14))
 (segment (start 153.924006 40.386) (end 154.051 40.259006) (width 0.4) (layer F.Cu) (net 14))
 (segment (start 149.520006 40.386) (end 153.924006 40.386) (width 0.4) (layer F.Cu) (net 14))
 (segment (start 149.482004 40.424002) (end 149.520006 40.386) (width 0.4) (layer F.Cu) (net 14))
 (segment (start 139.357198 40.424002) (end 149.482004 40.424002) (width 0.4) (layer F.Cu) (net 14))
 (segment (start 133.604 47.625) (end 133.604 46.1772) (width 0.4) (layer F.Cu) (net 14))
 (segment (start 133.604 46.1772) (end 139.357198 40.424002) (width 0.4) (layer F.Cu) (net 14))
 (via (at 184.403996 40.9448) (size 0.8) (drill 0.4) (layers F.Cu B.Cu) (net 14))
 (segment (start 184.404 40.944804) (end 184.403996 40.9448) (width 0.4) (layer B.Cu) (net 14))
 (segment (start 184.404 47.625) (end 184.404 40.944804) (width 0.4) (layer B.Cu) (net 14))
 (segment (start 183.838311 40.9448) (end 184.403996 40.9448) (width 0.4) (layer F.Cu) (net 14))
 (segment (start 181.0004 40.9448) (end 183.838311 40.9448) (width 0.4) (layer F.Cu) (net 14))
 (segment (start 154.051 40.386) (end 180.4416 40.386) (width 0.4) (layer F.Cu) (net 14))
 (segment (start 180.4416 40.386) (end 181.0004 40.9448) (width 0.4) (layer F.Cu) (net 14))
 (via (at 176.784 42.291) (size 0.8) (drill 0.4) (layers F.Cu B.Cu) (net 17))
 (segment (start 176.784 47.625) (end 176.784 42.291) (width 0.4) (layer B.Cu) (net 17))
 (segment (start 125.984 46.475) (end 125.984 47.625) (width 0.4) (layer B.Cu) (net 17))
 (segment (start 126.319998 46.139002) (end 125.984 46.475) (width 0.4) (layer B.Cu) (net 17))
 (segment (start 150.075998 46.139002) (end 126.319998 46.139002) (width 0.4) (layer B.Cu) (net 17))
 (segment (start 151.511 43.561) (end 151.511 44.704) (width 0.4) (layer B.Cu) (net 17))
 (segment (start 151.511 44.704) (end 150.075998 46.139002) (width 0.4) (layer B.Cu) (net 17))
 (segment (start 151.511 42.7482) (end 151.511 43.561) (width 0.4) (layer F.Cu) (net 17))
 (segment (start 152.2222 42.037) (end 151.511 42.7482) (width 0.4) (layer F.Cu) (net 17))
 (segment (start 160.274 42.037) (end 152.2222 42.037) (width 0.4) (layer F.Cu) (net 17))
 (segment (start 176.784 42.291) (end 160.528 42.291) (width 0.4) (layer F.Cu) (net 17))
 (segment (start 160.528 42.291) (end 160.274 42.037) (width 0.4) (layer F.Cu) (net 17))
 (segment (start 166.751 34.80963) (end 166.751 35.941) (width 0.4) (layer B.Cu) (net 10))
 (segment (start 164.25017 32.3088) (end 166.751 34.80963) (width 0.4) (layer B.Cu) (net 10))
 (segment (start 141.6304 32.3088) (end 164.25017 32.3088) (width 0.4) (layer B.Cu) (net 10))
 (segment (start 140.556599 31.234999) (end 141.6304 32.3088) (width 0.4) (layer B.Cu) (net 10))
 (segment (start 136.144 32.385) (end 137.294001 31.234999) (width 0.4) (layer B.Cu) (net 10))
 (segment (start 137.294001 31.234999) (end 140.556599 31.234999) (width 0.4) (layer B.Cu) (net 10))
 (segment (start 181.864 47.625) (end 181.864 39.751) (width 0.4) (layer B.Cu) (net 15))
 (segment (start 181.864 39.751) (end 181.737 39.624) (width 0.4) (layer B.Cu) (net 15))
 (via (at 181.737 39.624) (size 0.8) (drill 0.4) (layers F.Cu B.Cu) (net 15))
 (segment (start 148.971 39.62401) (end 148.97101 39.624) (width 0.4) (layer B.Cu) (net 15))
 (segment (start 181.737 39.624) (end 148.97101 39.624) (width 0.4) (layer F.Cu) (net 15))
 (segment (start 148.971 43.561) (end 148.971 39.62401) (width 0.4) (layer B.Cu) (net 15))
 (via (at 148.97101 39.624) (size 0.8) (drill 0.4) (layers F.Cu B.Cu) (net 15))
 (segment (start 148.405325 39.624) (end 148.97101 39.624) (width 0.4) (layer F.Cu) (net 15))
 (segment (start 137.6172 39.624) (end 148.405325 39.624) (width 0.4) (layer F.Cu) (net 15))
 (segment (start 131.064 47.625) (end 131.064 46.1772) (width 0.4) (layer F.Cu) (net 15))
 (segment (start 131.064 46.1772) (end 137.6172 39.624) (width 0.4) (layer F.Cu) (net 15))
 (segment (start 170.090999 35.141001) (end 169.291 35.941) (width 0.4) (layer F.Cu) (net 23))
 (segment (start 186.944 32.385) (end 186.944 33.4772) (width 0.4) (layer F.Cu) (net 23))
 (segment (start 185.1152 35.306) (end 173.5328 35.306) (width 0.4) (layer F.Cu) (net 23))
 (segment (start 173.5328 35.306) (end 172.967799 34.740999) (width 0.4) (layer F.Cu) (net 23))
 (segment (start 186.944 33.4772) (end 185.1152 35.306) (width 0.4) (layer F.Cu) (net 23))
 (segment (start 172.967799 34.740999) (end 170.491001 34.740999) (width 0.4) (layer F.Cu) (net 23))
 (segment (start 170.491001 34.740999) (end 170.090999 35.141001) (width 0.4) (layer F.Cu) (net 23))
 (segment (start 145.923006 45.084994) (end 146.431 44.577) (width 0.4) (layer B.Cu) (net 16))
 (segment (start 128.524 49.149) (end 128.27 49.403) (width 0.4) (layer B.Cu) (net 16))
 (segment (start 128.524 47.625) (end 128.524 49.149) (width 0.4) (layer B.Cu) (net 16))
 (segment (start 146.431 44.577) (end 146.431 43.561) (width 0.4) (layer B.Cu) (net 16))
 (segment (start 128.27 49.403) (end 124.714 49.403) (width 0.4) (layer B.Cu) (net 16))
 (segment (start 124.714 49.403) (end 124.206 48.895) (width 0.4) (layer B.Cu) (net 16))
 (segment (start 124.968006 45.084994) (end 145.923006 45.084994) (width 0.4) (layer B.Cu) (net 16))
 (segment (start 124.206 48.895) (end 124.206 45.847) (width 0.4) (layer B.Cu) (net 16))
 (segment (start 124.206 45.847) (end 124.968006 45.084994) (width 0.4) (layer B.Cu) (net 16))
 (segment (start 128.524 49.022) (end 128.524 47.625) (width 0.4) (layer F.Cu) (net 16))
 (segment (start 128.905 49.403) (end 128.524 49.022) (width 0.4) (layer F.Cu) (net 16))
 (segment (start 178.5874 49.403) (end 128.905 49.403) (width 0.4) (layer F.Cu) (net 16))
 (segment (start 179.324 47.625) (end 179.324 48.6664) (width 0.4) (layer F.Cu) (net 16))
 (segment (start 179.324 48.6664) (end 178.5874 49.403) (width 0.4) (layer F.Cu) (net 16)))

